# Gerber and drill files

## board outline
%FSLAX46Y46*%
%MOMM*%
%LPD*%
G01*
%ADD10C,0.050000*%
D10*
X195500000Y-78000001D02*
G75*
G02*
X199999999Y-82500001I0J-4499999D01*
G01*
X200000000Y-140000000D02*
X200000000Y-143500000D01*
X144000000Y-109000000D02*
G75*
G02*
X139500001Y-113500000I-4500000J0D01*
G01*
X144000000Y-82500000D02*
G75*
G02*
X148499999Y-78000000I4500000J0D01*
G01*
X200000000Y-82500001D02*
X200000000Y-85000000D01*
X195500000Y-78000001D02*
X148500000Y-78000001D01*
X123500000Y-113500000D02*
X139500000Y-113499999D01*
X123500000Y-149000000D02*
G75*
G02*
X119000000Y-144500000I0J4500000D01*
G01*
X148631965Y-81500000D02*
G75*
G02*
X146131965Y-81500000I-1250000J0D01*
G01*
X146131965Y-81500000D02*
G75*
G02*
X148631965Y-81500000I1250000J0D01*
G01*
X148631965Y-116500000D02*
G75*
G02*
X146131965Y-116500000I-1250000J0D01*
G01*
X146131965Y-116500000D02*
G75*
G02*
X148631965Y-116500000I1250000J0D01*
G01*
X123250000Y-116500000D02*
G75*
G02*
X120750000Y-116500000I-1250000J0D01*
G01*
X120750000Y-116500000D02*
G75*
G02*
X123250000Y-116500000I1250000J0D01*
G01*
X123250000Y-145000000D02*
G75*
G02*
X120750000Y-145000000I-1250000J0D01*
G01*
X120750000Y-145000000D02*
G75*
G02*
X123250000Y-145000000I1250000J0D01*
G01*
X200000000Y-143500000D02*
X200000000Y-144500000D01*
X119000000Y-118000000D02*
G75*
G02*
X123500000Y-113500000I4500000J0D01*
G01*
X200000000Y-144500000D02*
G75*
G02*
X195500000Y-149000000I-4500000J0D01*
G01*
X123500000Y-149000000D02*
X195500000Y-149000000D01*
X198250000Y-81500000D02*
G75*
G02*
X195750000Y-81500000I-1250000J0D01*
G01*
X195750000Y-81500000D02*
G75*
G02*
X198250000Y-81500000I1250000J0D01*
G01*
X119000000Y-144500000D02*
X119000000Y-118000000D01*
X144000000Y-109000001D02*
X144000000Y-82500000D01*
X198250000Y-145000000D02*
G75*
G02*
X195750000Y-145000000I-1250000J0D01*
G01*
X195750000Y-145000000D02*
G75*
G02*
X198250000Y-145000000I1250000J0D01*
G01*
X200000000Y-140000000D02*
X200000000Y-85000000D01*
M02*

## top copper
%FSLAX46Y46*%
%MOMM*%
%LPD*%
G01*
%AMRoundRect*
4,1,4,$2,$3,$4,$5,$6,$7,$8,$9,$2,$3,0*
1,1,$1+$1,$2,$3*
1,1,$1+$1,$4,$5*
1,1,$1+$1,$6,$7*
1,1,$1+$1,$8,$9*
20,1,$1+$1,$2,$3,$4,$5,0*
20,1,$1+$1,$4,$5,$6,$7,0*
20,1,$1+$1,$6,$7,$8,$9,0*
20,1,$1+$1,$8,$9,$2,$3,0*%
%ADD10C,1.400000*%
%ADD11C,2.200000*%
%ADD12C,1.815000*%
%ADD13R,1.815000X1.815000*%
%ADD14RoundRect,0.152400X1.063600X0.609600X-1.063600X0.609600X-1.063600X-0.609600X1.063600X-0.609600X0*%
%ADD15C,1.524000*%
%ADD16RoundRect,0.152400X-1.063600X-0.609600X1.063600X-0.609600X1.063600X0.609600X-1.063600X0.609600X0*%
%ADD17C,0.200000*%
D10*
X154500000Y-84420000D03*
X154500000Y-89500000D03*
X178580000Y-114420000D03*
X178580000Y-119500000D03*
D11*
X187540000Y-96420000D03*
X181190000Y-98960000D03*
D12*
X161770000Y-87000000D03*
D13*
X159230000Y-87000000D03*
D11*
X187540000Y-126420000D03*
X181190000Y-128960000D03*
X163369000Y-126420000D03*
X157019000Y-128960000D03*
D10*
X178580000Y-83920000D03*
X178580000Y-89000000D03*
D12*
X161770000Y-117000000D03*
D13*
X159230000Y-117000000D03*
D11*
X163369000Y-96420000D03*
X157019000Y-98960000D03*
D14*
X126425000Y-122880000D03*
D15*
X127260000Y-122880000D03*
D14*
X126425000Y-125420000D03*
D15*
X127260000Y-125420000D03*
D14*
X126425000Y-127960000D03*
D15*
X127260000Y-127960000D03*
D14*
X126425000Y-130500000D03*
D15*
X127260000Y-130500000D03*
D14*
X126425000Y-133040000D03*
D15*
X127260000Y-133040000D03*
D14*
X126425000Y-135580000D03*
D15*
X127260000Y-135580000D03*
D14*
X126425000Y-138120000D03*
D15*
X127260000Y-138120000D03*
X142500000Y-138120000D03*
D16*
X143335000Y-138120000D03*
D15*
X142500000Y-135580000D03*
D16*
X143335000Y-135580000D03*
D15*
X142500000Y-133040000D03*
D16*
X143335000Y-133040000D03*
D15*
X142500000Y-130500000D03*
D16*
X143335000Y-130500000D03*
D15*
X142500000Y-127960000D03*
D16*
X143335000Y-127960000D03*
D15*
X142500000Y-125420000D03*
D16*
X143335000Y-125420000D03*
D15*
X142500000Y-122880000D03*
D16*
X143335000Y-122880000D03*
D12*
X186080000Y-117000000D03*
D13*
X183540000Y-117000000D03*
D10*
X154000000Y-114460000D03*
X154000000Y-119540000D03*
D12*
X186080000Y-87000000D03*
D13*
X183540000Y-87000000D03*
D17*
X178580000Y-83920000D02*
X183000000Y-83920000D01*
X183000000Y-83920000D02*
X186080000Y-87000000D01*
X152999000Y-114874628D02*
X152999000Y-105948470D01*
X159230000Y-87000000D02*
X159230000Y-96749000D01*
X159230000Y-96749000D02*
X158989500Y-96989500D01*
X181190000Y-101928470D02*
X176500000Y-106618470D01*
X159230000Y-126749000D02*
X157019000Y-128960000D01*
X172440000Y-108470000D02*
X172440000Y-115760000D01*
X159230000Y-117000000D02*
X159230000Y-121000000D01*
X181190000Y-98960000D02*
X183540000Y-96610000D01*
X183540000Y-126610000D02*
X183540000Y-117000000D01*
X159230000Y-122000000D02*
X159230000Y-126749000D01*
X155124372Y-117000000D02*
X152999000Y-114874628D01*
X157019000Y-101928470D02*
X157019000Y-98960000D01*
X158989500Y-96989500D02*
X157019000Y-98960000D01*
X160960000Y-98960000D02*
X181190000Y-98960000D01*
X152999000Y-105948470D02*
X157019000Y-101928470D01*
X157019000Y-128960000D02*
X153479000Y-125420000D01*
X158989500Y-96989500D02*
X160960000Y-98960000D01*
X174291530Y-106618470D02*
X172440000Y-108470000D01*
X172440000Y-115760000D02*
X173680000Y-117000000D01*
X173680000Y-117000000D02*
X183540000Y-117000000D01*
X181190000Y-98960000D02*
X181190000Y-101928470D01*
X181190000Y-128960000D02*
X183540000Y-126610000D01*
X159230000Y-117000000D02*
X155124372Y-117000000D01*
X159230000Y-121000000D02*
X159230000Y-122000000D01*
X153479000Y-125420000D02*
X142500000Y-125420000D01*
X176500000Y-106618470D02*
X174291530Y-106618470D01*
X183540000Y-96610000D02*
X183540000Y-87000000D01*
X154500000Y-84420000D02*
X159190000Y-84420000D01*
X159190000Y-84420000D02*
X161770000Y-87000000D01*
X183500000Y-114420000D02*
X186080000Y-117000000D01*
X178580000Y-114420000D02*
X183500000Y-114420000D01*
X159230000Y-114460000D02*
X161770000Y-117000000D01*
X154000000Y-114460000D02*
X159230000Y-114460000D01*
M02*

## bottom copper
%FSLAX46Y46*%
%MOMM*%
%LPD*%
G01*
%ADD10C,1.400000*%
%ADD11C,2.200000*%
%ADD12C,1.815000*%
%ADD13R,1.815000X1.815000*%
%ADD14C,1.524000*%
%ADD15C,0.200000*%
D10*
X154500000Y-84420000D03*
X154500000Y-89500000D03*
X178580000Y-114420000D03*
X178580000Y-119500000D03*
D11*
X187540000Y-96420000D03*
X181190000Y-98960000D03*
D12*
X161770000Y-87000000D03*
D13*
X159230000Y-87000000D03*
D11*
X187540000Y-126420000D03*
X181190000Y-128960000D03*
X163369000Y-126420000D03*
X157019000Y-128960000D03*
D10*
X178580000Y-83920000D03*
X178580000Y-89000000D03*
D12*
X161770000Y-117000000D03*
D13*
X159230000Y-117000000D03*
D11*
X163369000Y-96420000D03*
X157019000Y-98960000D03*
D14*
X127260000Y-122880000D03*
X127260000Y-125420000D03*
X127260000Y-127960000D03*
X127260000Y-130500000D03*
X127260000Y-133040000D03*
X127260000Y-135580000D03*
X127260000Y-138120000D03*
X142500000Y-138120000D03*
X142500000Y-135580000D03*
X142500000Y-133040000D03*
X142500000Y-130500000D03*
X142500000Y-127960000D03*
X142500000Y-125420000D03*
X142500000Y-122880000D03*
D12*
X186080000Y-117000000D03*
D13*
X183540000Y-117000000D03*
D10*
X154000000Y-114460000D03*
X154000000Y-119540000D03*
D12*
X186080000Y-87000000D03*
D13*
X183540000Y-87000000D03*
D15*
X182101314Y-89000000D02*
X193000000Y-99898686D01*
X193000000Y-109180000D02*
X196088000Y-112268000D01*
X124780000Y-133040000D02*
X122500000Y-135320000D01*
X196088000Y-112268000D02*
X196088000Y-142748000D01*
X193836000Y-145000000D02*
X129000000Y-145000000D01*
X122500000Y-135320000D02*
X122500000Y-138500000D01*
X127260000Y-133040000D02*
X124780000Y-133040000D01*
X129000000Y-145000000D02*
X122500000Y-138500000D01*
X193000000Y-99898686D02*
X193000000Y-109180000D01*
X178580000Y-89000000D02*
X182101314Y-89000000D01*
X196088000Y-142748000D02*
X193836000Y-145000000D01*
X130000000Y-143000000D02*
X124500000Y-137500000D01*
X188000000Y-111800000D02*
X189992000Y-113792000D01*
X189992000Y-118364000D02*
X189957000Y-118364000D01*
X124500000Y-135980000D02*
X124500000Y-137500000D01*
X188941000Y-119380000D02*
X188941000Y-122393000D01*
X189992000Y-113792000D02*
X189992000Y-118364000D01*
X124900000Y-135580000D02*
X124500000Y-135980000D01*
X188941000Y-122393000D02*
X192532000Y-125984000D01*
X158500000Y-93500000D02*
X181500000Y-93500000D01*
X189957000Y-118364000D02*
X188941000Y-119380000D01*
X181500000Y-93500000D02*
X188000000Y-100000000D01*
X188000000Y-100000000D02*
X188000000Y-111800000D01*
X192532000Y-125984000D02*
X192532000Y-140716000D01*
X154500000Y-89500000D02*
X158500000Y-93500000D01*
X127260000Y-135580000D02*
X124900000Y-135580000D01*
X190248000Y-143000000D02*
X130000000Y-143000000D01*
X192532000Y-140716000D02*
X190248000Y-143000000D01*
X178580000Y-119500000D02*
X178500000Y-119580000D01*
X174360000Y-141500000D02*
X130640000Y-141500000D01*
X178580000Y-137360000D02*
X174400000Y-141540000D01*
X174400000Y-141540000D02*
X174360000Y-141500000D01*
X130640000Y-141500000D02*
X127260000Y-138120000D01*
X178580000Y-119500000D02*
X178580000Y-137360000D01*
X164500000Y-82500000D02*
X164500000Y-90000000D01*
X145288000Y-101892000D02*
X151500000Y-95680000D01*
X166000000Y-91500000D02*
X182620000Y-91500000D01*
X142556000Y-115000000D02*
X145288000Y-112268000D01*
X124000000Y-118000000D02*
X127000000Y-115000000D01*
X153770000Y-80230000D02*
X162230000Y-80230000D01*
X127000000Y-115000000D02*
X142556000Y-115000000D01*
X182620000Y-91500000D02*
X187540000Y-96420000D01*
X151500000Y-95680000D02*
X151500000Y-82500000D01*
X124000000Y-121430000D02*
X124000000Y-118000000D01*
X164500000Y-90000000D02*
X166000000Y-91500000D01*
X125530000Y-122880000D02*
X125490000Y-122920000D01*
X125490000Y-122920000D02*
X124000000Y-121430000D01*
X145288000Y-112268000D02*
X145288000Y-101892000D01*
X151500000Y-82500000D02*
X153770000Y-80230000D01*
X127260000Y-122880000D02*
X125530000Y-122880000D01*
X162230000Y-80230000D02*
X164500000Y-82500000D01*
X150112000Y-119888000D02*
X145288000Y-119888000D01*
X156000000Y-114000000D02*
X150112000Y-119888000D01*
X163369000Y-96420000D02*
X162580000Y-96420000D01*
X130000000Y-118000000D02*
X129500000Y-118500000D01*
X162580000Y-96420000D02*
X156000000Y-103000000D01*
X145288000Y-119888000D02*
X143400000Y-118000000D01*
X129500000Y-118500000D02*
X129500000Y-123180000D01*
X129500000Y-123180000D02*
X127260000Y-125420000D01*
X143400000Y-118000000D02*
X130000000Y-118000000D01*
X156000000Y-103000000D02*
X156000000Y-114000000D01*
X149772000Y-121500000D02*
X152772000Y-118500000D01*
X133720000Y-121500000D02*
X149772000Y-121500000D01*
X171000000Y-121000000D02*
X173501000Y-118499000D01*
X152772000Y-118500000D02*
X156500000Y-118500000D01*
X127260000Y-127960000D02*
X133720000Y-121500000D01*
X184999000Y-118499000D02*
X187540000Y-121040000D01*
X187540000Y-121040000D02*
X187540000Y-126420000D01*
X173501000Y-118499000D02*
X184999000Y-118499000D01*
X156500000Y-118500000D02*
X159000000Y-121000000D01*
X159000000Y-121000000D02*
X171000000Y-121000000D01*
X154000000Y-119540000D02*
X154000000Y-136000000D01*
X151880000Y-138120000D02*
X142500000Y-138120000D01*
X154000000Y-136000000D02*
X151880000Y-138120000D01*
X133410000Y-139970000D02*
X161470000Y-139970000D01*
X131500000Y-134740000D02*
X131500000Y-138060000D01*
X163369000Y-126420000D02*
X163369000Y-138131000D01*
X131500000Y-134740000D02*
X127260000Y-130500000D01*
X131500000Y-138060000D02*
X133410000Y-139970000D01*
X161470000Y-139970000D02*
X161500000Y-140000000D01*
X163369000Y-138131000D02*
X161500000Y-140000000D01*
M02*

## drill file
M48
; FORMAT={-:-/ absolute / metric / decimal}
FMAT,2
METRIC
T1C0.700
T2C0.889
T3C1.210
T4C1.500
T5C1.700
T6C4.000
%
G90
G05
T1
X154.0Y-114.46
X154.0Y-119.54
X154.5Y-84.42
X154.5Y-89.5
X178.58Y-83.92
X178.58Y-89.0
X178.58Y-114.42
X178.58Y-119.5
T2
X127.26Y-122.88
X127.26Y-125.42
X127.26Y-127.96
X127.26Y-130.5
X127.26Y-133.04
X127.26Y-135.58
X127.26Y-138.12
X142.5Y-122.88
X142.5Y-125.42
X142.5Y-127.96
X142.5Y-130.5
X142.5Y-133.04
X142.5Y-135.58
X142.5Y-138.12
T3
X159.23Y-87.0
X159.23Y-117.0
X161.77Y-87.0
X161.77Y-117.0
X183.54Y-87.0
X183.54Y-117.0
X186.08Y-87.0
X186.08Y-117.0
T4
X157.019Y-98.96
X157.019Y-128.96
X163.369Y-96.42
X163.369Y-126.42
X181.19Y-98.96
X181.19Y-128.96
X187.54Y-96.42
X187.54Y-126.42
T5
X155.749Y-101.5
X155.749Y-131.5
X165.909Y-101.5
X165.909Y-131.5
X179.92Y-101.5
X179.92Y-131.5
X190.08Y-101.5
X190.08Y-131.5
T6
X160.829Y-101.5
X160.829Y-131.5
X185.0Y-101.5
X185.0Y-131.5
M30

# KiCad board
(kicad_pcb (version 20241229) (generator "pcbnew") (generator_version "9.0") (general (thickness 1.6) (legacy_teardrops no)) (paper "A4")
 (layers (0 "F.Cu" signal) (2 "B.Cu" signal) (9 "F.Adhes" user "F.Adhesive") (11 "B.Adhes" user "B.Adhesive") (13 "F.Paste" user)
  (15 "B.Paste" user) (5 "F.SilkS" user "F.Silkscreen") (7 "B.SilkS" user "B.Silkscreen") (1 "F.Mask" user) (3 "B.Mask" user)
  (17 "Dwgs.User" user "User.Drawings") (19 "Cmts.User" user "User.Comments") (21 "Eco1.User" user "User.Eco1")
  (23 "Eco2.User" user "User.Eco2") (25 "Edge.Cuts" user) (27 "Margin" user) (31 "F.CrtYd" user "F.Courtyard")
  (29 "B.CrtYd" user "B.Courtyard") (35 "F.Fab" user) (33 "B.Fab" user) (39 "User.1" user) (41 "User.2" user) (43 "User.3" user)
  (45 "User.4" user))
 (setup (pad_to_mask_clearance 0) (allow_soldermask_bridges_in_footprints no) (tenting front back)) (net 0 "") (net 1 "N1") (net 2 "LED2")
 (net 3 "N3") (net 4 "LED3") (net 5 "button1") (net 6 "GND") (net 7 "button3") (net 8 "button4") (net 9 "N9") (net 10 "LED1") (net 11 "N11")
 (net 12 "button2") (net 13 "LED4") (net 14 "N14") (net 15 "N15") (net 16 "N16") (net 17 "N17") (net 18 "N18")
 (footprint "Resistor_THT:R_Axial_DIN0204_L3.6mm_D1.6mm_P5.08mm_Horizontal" (layer "F.Cu") (at 154.5 84.42 -90)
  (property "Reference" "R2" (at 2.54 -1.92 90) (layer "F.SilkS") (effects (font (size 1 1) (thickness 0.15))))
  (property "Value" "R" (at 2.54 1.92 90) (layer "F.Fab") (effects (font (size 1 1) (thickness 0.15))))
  (pad "1" thru_hole circle (at 0 0 270) (size 1.4 1.4) (drill 0.7) (layers "*.Cu" "*.Mask") (remove_unused_layers no) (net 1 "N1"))
  (pad "2" thru_hole circle (at 5.08 0 270) (size 1.4 1.4) (drill 0.7) (layers "*.Cu" "*.Mask") (remove_unused_layers no) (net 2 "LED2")))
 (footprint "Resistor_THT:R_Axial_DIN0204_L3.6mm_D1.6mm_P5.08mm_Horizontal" (layer "F.Cu") (at 178.58 114.42 -90)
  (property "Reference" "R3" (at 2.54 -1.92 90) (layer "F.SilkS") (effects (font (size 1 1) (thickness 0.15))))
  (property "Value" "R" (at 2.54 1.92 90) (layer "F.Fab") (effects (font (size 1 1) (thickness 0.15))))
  (pad "1" thru_hole circle (at 0 0 270) (size 1.4 1.4) (drill 0.7) (layers "*.Cu" "*.Mask") (remove_unused_layers no) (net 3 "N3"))
  (pad "2" thru_hole circle (at 5.08 0 270) (size 1.4 1.4) (drill 0.7) (layers "*.Cu" "*.Mask") (remove_unused_layers no) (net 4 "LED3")))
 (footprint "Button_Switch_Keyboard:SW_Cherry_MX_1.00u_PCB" (layer "F.Cu") (at 187.54 96.42)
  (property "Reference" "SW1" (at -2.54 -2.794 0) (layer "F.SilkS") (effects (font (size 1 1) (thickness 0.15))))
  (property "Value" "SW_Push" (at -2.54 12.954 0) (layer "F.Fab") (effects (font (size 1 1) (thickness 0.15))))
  (pad "" np_thru_hole circle (at -7.62 5.08) (size 1.7 1.7) (drill 1.7) (layers "*.Cu" "*.Mask"))
  (pad "" np_thru_hole circle (at -2.54 5.08) (size 4 4) (drill 4) (layers "*.Cu" "*.Mask"))
  (pad "" np_thru_hole circle (at 2.54 5.08) (size 1.7 1.7) (drill 1.7) (layers "*.Cu" "*.Mask"))
  (pad "1" thru_hole circle (at 0 0) (size 2.2 2.2) (drill 1.5) (layers "*.Cu" "*.Mask") (remove_unused_layers no) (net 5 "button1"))
  (pad "2" thru_hole circle (at -6.35 2.54) (size 2.2 2.2) (drill 1.5) (layers "*.Cu" "*.Mask") (remove_unused_layers no) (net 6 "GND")))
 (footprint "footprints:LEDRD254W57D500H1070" (layer "F.Cu") (at 160.5 87)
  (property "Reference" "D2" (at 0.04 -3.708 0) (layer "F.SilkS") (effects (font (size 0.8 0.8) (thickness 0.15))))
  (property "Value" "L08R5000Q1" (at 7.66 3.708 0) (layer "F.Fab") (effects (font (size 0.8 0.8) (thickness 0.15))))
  (pad "A" thru_hole circle (at 1.27 0) (size 1.815 1.815) (drill 1.21) (layers "*.Cu" "*.Mask") (remove_unused_layers no) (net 1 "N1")
   (solder_mask_margin 0.102))
  (pad "C" thru_hole rect (at -1.27 0) (size 1.815 1.815) (drill 1.21) (layers "*.Cu" "*.Mask") (remove_unused_layers no) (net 6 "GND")
   (solder_mask_margin 0.102)))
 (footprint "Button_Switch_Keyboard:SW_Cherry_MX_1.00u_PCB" (layer "F.Cu") (at 187.54 126.42)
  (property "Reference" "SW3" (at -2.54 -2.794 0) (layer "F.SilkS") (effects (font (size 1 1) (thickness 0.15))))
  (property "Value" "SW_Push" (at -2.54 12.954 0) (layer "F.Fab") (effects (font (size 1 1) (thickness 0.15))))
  (pad "" np_thru_hole circle (at -7.62 5.08) (size 1.7 1.7) (drill 1.7) (layers "*.Cu" "*.Mask"))
  (pad "" np_thru_hole circle (at -2.54 5.08) (size 4 4) (drill 4) (layers "*.Cu" "*.Mask"))
  (pad "" np_thru_hole circle (at 2.54 5.08) (size 1.7 1.7) (drill 1.7) (layers "*.Cu" "*.Mask"))
  (pad "1" thru_hole circle (at 0 0) (size 2.2 2.2) (drill 1.5) (layers "*.Cu" "*.Mask") (remove_unused_layers no) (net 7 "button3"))
  (pad "2" thru_hole circle (at -6.35 2.54) (size 2.2 2.2) (drill 1.5) (layers "*.Cu" "*.Mask") (remove_unused_layers no) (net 6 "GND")))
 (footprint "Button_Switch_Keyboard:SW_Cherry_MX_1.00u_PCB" (layer "F.Cu") (at 163.369 126.42)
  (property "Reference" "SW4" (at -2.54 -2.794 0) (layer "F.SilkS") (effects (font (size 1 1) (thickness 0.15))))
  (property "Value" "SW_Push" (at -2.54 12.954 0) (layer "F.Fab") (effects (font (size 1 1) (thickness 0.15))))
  (pad "" np_thru_hole circle (at -7.62 5.08) (size 1.7 1.7) (drill 1.7) (layers "*.Cu" "*.Mask"))
  (pad "" np_thru_hole circle (at -2.54 5.08) (size 4 4) (drill 4) (layers "*.Cu" "*.Mask"))
  (pad "" np_thru_hole circle (at 2.54 5.08) (size 1.7 1.7) (drill 1.7) (layers "*.Cu" "*.Mask"))
  (pad "1" thru_hole circle (at 0 0) (size 2.2 2.2) (drill 1.5) (layers "*.Cu" "*.Mask") (remove_unused_layers no) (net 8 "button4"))
  (pad "2" thru_hole circle (at -6.35 2.54) (size 2.2 2.2) (drill 1.5) (layers "*.Cu" "*.Mask") (remove_unused_layers no) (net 6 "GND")))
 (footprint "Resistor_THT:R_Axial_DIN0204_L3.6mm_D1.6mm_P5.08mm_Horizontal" (layer "F.Cu") (at 178.58 83.92 -90)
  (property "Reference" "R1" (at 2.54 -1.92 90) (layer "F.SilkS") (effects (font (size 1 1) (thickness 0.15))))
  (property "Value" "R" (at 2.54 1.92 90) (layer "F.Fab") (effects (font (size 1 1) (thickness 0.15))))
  (pad "1" thru_hole circle (at 0 0 270) (size 1.4 1.4) (drill 0.7) (layers "*.Cu" "*.Mask") (remove_unused_layers no) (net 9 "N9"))
  (pad "2" thru_hole circle (at 5.08 0 270) (size 1.4 1.4) (drill 0.7) (layers "*.Cu" "*.Mask") (remove_unused_layers no) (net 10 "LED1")))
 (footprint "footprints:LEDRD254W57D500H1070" (layer "F.Cu") (at 160.5 117)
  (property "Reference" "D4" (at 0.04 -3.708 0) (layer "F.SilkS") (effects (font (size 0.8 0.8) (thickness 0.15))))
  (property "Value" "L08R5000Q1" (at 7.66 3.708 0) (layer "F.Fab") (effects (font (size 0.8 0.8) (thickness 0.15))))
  (pad "A" thru_hole circle (at 1.27 0) (size 1.815 1.815) (drill 1.21) (layers "*.Cu" "*.Mask") (remove_unused_layers no) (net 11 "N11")
   (solder_mask_margin 0.102))
  (pad "C" thru_hole rect (at -1.27 0) (size 1.815 1.815) (drill 1.21) (layers "*.Cu" "*.Mask") (remove_unused_layers no) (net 6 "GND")
   (solder_mask_margin 0.102)))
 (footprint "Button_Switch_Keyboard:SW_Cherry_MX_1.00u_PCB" (layer "F.Cu") (at 163.369 96.42)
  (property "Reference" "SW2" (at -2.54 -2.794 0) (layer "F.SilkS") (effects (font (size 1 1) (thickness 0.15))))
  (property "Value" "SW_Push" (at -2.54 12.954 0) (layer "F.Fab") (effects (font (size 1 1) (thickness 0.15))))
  (pad "" np_thru_hole circle (at -7.62 5.08) (size 1.7 1.7) (drill 1.7) (layers "*.Cu" "*.Mask"))
  (pad "" np_thru_hole circle (at -2.54 5.08) (size 4 4) (drill 4) (layers "*.Cu" "*.Mask"))
  (pad "" np_thru_hole circle (at 2.54 5.08) (size 1.7 1.7) (drill 1.7) (layers "*.Cu" "*.Mask"))
  (pad "1" thru_hole circle (at 0 0) (size 2.2 2.2) (drill 1.5) (layers "*.Cu" "*.Mask") (remove_unused_layers no) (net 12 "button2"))
  (pad "2" thru_hole circle (at -6.35 2.54) (size 2.2 2.2) (drill 1.5) (layers "*.Cu" "*.Mask") (remove_unused_layers no) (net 6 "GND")))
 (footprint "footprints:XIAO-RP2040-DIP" (layer "F.Cu") (at 134.88 130.5)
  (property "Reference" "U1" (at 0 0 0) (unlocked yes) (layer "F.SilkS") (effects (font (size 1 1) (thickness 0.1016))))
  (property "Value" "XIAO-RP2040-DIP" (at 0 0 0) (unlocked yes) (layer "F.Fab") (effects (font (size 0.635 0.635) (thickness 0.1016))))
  (pad "1" smd roundrect (at -8.455 -7.62 180) (size 2.432 1.524) (layers "F.Cu" "F.Mask") (roundrect_rratio 0.1) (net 5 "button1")
   (thermal_bridge_angle 45))
  (pad "1" thru_hole circle (at -7.62 -7.62 180) (size 1.524 1.524) (drill 0.889) (layers "*.Cu" "*.Mask") (remove_unused_layers no)
   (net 5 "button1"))
  (pad "2" smd roundrect (at -8.455 -5.08 180) (size 2.432 1.524) (layers "F.Cu" "F.Mask") (roundrect_rratio 0.1) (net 12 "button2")
   (thermal_bridge_angle 45))
  (pad "2" thru_hole circle (at -7.62 -5.08 180) (size 1.524 1.524) (drill 0.889) (layers "*.Cu" "*.Mask") (remove_unused_layers no)
   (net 12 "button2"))
  (pad "3" smd roundrect (at -8.455 -2.54 180) (size 2.432 1.524) (layers "F.Cu" "F.Mask") (roundrect_rratio 0.1) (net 7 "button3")
   (thermal_bridge_angle 45))
  (pad "3" thru_hole circle (at -7.62 -2.54 180) (size 1.524 1.524) (drill 0.889) (layers "*.Cu" "*.Mask") (remove_unused_layers no)
   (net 7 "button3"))
  (pad "4" smd roundrect (at -8.455 0 180) (size 2.432 1.524) (layers "F.Cu" "F.Mask") (roundrect_rratio 0.1) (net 8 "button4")
   (thermal_bridge_angle 45))
  (pad "4" thru_hole circle (at -7.62 0 180) (size 1.524 1.524) (drill 0.889) (layers "*.Cu" "*.Mask") (remove_unused_layers no)
   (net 8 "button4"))
  (pad "5" smd roundrect (at -8.455 2.54 180) (size 2.432 1.524) (layers "F.Cu" "F.Mask") (roundrect_rratio 0.1) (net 10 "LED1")
   (thermal_bridge_angle 45))
  (pad "5" thru_hole circle (at -7.62 2.54 180) (size 1.524 1.524) (drill 0.889) (layers "*.Cu" "*.Mask") (remove_unused_layers no)
   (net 10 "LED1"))
  (pad "6" smd roundrect (at -8.455 5.08 180) (size 2.432 1.524) (layers "F.Cu" "F.Mask") (roundrect_rratio 0.1) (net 2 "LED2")
   (thermal_bridge_angle 45))
  (pad "6" thru_hole circle (at -7.62 5.08 180) (size 1.524 1.524) (drill 0.889) (layers "*.Cu" "*.Mask") (remove_unused_layers no)
   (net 2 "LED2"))
  (pad "7" smd roundrect (at -8.455 7.62 180) (size 2.432 1.524) (layers "F.Cu" "F.Mask") (roundrect_rratio 0.1) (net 4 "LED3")
   (thermal_bridge_angle 45))
  (pad "7" thru_hole circle (at -7.62 7.62 180) (size 1.524 1.524) (drill 0.889) (layers "*.Cu" "*.Mask") (remove_unused_layers no)
   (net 4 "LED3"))
  (pad "8" thru_hole circle (at 7.62 7.62) (size 1.524 1.524) (drill 0.889) (layers "*.Cu" "*.Mask") (remove_unused_layers no)
   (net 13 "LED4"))
  (pad "8" smd roundrect (at 8.455 7.62) (size 2.432 1.524) (layers "F.Cu" "F.Mask") (roundrect_rratio 0.1) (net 13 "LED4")
   (thermal_bridge_angle 45))
  (pad "9" thru_hole circle (at 7.62 5.08) (size 1.524 1.524) (drill 0.889) (layers "*.Cu" "*.Mask") (remove_unused_layers no)
   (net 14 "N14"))
  (pad "9" smd roundrect (at 8.455 5.08) (size 2.432 1.524) (layers "F.Cu" "F.Mask") (roundrect_rratio 0.1) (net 14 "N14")
   (thermal_bridge_angle 45))
  (pad "10" thru_hole circle (at 7.62 2.54) (size 1.524 1.524) (drill 0.889) (layers "*.Cu" "*.Mask") (remove_unused_layers no)
   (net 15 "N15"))
  (pad "10" smd roundrect (at 8.455 2.54) (size 2.432 1.524) (layers "F.Cu" "F.Mask") (roundrect_rratio 0.1) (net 15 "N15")
   (thermal_bridge_angle 45))
  (pad "11" thru_hole circle (at 7.62 0) (size 1.524 1.524) (drill 0.889) (layers "*.Cu" "*.Mask") (remove_unused_layers no) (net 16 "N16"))
  (pad "11" smd roundrect (at 8.455 0) (size 2.432 1.524) (layers "F.Cu" "F.Mask") (roundrect_rratio 0.1) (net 16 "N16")
   (thermal_bridge_angle 45))
  (pad "12" thru_hole circle (at 7.62 -2.54) (size 1.524 1.524) (drill 0.889) (layers "*.Cu" "*.Mask") (remove_unused_layers no)
   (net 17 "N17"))
  (pad "12" smd roundrect (at 8.455 -2.54) (size 2.432 1.524) (layers "F.Cu" "F.Mask") (roundrect_rratio 0.1) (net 17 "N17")
   (thermal_bridge_angle 45))
  (pad "13" thru_hole circle (at 7.62 -5.08) (size 1.524 1.524) (drill 0.889) (layers "*.Cu" "*.Mask") (remove_unused_layers no)
   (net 6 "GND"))
  (pad "13" smd roundrect (at 8.455 -5.08) (size 2.432 1.524) (layers "F.Cu" "F.Mask") (roundrect_rratio 0.1) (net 6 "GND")
   (thermal_bridge_angle 45))
  (pad "14" thru_hole circle (at 7.62 -7.62) (size 1.524 1.524) (drill 0.889) (layers "*.Cu" "*.Mask") (remove_unused_layers no)
   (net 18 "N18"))
  (pad "14" smd roundrect (at 8.455 -7.62) (size 2.432 1.524) (layers "F.Cu" "F.Mask") (roundrect_rratio 0.1) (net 18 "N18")
   (thermal_bridge_angle 45)))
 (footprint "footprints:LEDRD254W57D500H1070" (layer "F.Cu") (at 184.81 117)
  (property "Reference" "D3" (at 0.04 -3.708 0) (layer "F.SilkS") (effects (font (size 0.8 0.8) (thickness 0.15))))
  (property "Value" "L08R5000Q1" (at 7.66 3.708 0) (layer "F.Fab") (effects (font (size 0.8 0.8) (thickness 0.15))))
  (pad "A" thru_hole circle (at 1.27 0) (size 1.815 1.815) (drill 1.21) (layers "*.Cu" "*.Mask") (remove_unused_layers no) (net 3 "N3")
   (solder_mask_margin 0.102))
  (pad "C" thru_hole rect (at -1.27 0) (size 1.815 1.815) (drill 1.21) (layers "*.Cu" "*.Mask") (remove_unused_layers no) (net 6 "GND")
   (solder_mask_margin 0.102)))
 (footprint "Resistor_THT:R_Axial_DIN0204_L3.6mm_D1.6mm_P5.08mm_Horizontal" (layer "F.Cu") (at 154 114.46 -90)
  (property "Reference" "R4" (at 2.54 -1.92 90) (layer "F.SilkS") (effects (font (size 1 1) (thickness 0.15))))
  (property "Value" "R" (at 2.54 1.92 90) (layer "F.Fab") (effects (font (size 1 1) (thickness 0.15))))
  (pad "1" thru_hole circle (at 0 0 270) (size 1.4 1.4) (drill 0.7) (layers "*.Cu" "*.Mask") (remove_unused_layers no) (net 11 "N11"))
  (pad "2" thru_hole circle (at 5.08 0 270) (size 1.4 1.4) (drill 0.7) (layers "*.Cu" "*.Mask") (remove_unused_layers no) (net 13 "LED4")))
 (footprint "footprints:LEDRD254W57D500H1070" (layer "F.Cu") (at 184.81 87)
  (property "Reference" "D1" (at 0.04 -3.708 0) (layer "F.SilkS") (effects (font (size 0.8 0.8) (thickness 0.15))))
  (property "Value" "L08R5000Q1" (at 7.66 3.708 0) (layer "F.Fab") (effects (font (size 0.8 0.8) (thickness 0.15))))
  (pad "A" thru_hole circle (at 1.27 0) (size 1.815 1.815) (drill 1.21) (layers "*.Cu" "*.Mask") (remove_unused_layers no) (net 9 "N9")
   (solder_mask_margin 0.102))
  (pad "C" thru_hole rect (at -1.27 0) (size 1.815 1.815) (drill 1.21) (layers "*.Cu" "*.Mask") (remove_unused_layers no) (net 6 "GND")
   (solder_mask_margin 0.102)))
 (gr_arc (start 195.5 78.000001) (mid 198.681981 79.31802) (end 200 82.500001) (stroke (width 0.05) (type default)) (layer "Edge.Cuts"))
 (gr_line (start 200 140) (end 200 143.5) (stroke (width 0.05) (type default)) (layer "Edge.Cuts"))
 (gr_arc (start 144 109) (mid 142.681982 112.181986) (end 139.500001 113.499999) (stroke (width 0.05) (type default)) (layer "Edge.Cuts"))
 (gr_arc (start 144 82.5) (mid 145.31802 79.318026) (end 148.499999 78.000001) (stroke (width 0.05) (type default)) (layer "Edge.Cuts"))
 (gr_line (start 200 82.500001) (end 200 85) (stroke (width 0.05) (type default)) (layer "Edge.Cuts"))
 (gr_line (start 195.5 78.000001) (end 148.5 78.000001) (stroke (width 0.05) (type default)) (layer "Edge.Cuts"))
 (gr_line (start 123.5 113.5) (end 139.5 113.499999) (stroke (width 0.05) (type default)) (layer "Edge.Cuts"))
 (gr_arc (start 123.5 149) (mid 120.318019 147.681981) (end 119 144.5) (stroke (width 0.05) (type default)) (layer "Edge.Cuts"))
 (gr_circle (center 147.381965 81.5) (end 148.631965 81.5) (stroke (width 0.05) (type solid)) (fill no) (layer "Edge.Cuts"))
 (gr_circle (center 147.381965 116.5) (end 148.631965 116.5) (stroke (width 0.05) (type solid)) (fill no) (layer "Edge.Cuts"))
 (gr_circle (center 122 116.5) (end 123.25 116.5) (stroke (width 0.05) (type solid)) (fill no) (layer "Edge.Cuts"))
 (gr_circle (center 122 145) (end 123.25 145) (stroke (width 0.05) (type solid)) (fill no) (layer "Edge.Cuts"))
 (gr_line (start 200 143.5) (end 200 144.5) (stroke (width 0.05) (type default)) (layer "Edge.Cuts"))
 (gr_arc (start 119 118) (mid 120.31802 114.81802) (end 123.5 113.5) (stroke (width 0.05) (type default)) (layer "Edge.Cuts"))
 (gr_arc (start 200 144.5) (mid 198.681981 147.681981) (end 195.5 149) (stroke (width 0.05) (type default)) (layer "Edge.Cuts"))
 (gr_line (start 123.5 149) (end 195.5 149) (stroke (width 0.05) (type default)) (layer "Edge.Cuts"))
 (gr_circle (center 197 81.5) (end 198.25 81.5) (stroke (width 0.05) (type solid)) (fill no) (layer "Edge.Cuts"))
 (gr_line (start 119 144.5) (end 119 118) (stroke (width 0.05) (type default)) (layer "Edge.Cuts"))
 (gr_line (start 144 109.000001) (end 144 82.5) (stroke (width 0.05) (type default)) (layer "Edge.Cuts"))
 (gr_circle (center 197 145) (end 198.25 145) (stroke (width 0.05) (type solid)) (fill no) (layer "Edge.Cuts"))
 (gr_line (start 200 140) (end 200 85) (stroke (width 0.05) (type solid)) (layer "Edge.Cuts"))
 (segment (start 178.58 83.92) (end 183 83.92) (width 0.2) (layer "F.Cu") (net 9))
 (segment (start 183 83.92) (end 186.08 87) (width 0.2) (layer "F.Cu") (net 9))
 (segment (start 152.999 114.874628) (end 152.999 105.94847) (width 0.2) (layer "F.Cu") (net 6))
 (segment (start 159.23 87) (end 159.23 96.749) (width 0.2) (layer "F.Cu") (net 6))
 (segment (start 159.23 96.749) (end 158.9895 96.9895) (width 0.2) (layer "F.Cu") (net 6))
 (segment (start 181.19 101.92847) (end 176.5 106.61847) (width 0.2) (layer "F.Cu") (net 6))
 (segment (start 159.23 126.749) (end 157.019 128.96) (width 0.2) (layer "F.Cu") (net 6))
 (segment (start 172.44 108.47) (end 172.44 115.76) (width 0.2) (layer "F.Cu") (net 6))
 (segment (start 159.23 117) (end 159.23 121) (width 0.2) (layer "F.Cu") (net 6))
 (segment (start 181.19 98.96) (end 183.54 96.61) (width 0.2) (layer "F.Cu") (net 6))
 (segment (start 183.54 126.61) (end 183.54 117) (width 0.2) (layer "F.Cu") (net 6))
 (segment (start 159.23 122) (end 159.23 126.749) (width 0.2) (layer "F.Cu") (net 6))
 (segment (start 155.124372 117) (end 152.999 114.874628) (width 0.2) (layer "F.Cu") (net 6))
 (segment (start 157.019 101.92847) (end 157.019 98.96) (width 0.2) (layer "F.Cu") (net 6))
 (segment (start 158.9895 96.9895) (end 157.019 98.96) (width 0.2) (layer "F.Cu") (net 6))
 (segment (start 160.96 98.96) (end 181.19 98.96) (width 0.2) (layer "F.Cu") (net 6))
 (segment (start 152.999 105.94847) (end 157.019 101.92847) (width 0.2) (layer "F.Cu") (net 6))
 (segment (start 157.019 128.96) (end 153.479 125.42) (width 0.2) (layer "F.Cu") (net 6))
 (segment (start 158.9895 96.9895) (end 160.96 98.96) (width 0.2) (layer "F.Cu") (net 6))
 (segment (start 174.29153 106.61847) (end 172.44 108.47) (width 0.2) (layer "F.Cu") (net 6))
 (segment (start 172.44 115.76) (end 173.68 117) (width 0.2) (layer "F.Cu") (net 6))
 (segment (start 173.68 117) (end 183.54 117) (width 0.2) (layer "F.Cu") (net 6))
 (segment (start 181.19 98.96) (end 181.19 101.92847) (width 0.2) (layer "F.Cu") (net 6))
 (segment (start 181.19 128.96) (end 183.54 126.61) (width 0.2) (layer "F.Cu") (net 6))
 (segment (start 159.23 117) (end 155.124372 117) (width 0.2) (layer "F.Cu") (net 6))
 (segment (start 159.23 121) (end 159.23 122) (width 0.2) (layer "F.Cu") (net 6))
 (segment (start 153.479 125.42) (end 142.5 125.42) (width 0.2) (layer "F.Cu") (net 6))
 (segment (start 176.5 106.61847) (end 174.29153 106.61847) (width 0.2) (layer "F.Cu") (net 6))
 (segment (start 183.54 96.61) (end 183.54 87) (width 0.2) (layer "F.Cu") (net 6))
 (segment (start 154.5 84.42) (end 159.19 84.42) (width 0.2) (layer "F.Cu") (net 1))
 (segment (start 159.19 84.42) (end 161.77 87) (width 0.2) (layer "F.Cu") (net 1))
 (segment (start 183.5 114.42) (end 186.08 117) (width 0.2) (layer "F.Cu") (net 3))
 (segment (start 178.58 114.42) (end 183.5 114.42) (width 0.2) (layer "F.Cu") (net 3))
 (segment (start 182.101314 89) (end 193 99.898686) (width 0.2) (layer "B.Cu") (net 10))
 (segment (start 193 109.18) (end 196.088 112.268) (width 0.2) (layer "B.Cu") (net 10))
 (segment (start 124.78 133.04) (end 122.5 135.32) (width 0.2) (layer "B.Cu") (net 10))
 (segment (start 196.088 112.268) (end 196.088 142.748) (width 0.2) (layer "B.Cu") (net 10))
 (segment (start 193.836 145) (end 129 145) (width 0.2) (layer "B.Cu") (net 10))
 (segment (start 122.5 135.32) (end 122.5 138.5) (width 0.2) (layer "B.Cu") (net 10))
 (segment (start 127.26 133.04) (end 124.78 133.04) (width 0.2) (layer "B.Cu") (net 10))
 (segment (start 129 145) (end 122.5 138.5) (width 0.2) (layer "B.Cu") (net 10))
 (segment (start 193 99.898686) (end 193 109.18) (width 0.2) (layer "B.Cu") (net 10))
 (segment (start 178.58 89) (end 182.101314 89) (width 0.2) (layer "B.Cu") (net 10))
 (segment (start 196.088 142.748) (end 193.836 145) (width 0.2) (layer "B.Cu") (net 10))
 (segment (start 130 143) (end 124.5 137.5) (width 0.2) (layer "B.Cu") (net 2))
 (segment (start 188 111.8) (end 189.992 113.792) (width 0.2) (layer "B.Cu") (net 2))
 (segment (start 189.992 118.364) (end 189.957 118.364) (width 0.2) (layer "B.Cu") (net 2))
 (segment (start 124.5 135.98) (end 124.5 137.5) (width 0.2) (layer "B.Cu") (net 2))
 (segment (start 188.941 119.38) (end 188.941 122.393) (width 0.2) (layer "B.Cu") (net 2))
 (segment (start 189.992 113.792) (end 189.992 118.364) (width 0.2) (layer "B.Cu") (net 2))
 (segment (start 124.9 135.58) (end 124.5 135.98) (width 0.2) (layer "B.Cu") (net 2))
 (segment (start 188.941 122.393) (end 192.532 125.984) (width 0.2) (layer "B.Cu") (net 2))
 (segment (start 158.5 93.5) (end 181.5 93.5) (width 0.2) (layer "B.Cu") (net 2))
 (segment (start 189.957 118.364) (end 188.941 119.38) (width 0.2) (layer "B.Cu") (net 2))
 (segment (start 181.5 93.5) (end 188 100) (width 0.2) (layer "B.Cu") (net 2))
 (segment (start 188 100) (end 188 111.8) (width 0.2) (layer "B.Cu") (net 2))
 (segment (start 192.532 125.984) (end 192.532 140.716) (width 0.2) (layer "B.Cu") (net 2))
 (segment (start 154.5 89.5) (end 158.5 93.5) (width 0.2) (layer "B.Cu") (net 2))
 (segment (start 127.26 135.58) (end 124.9 135.58) (width 0.2) (layer "B.Cu") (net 2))
 (segment (start 190.248 143) (end 130 143) (width 0.2) (layer "B.Cu") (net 2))
 (segment (start 192.532 140.716) (end 190.248 143) (width 0.2) (layer "B.Cu") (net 2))
 (segment (start 178.58 119.5) (end 178.5 119.58) (width 0.2) (layer "B.Cu") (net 4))
 (segment (start 174.36 141.5) (end 130.64 141.5) (width 0.2) (layer "B.Cu") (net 4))
 (segment (start 178.58 137.36) (end 174.4 141.54) (width 0.2) (layer "B.Cu") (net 4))
 (segment (start 174.4 141.54) (end 174.36 141.5) (width 0.2) (layer "B.Cu") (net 4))
 (segment (start 130.64 141.5) (end 127.26 138.12) (width 0.2) (layer "B.Cu") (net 4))
 (segment (start 178.58 119.5) (end 178.58 137.36) (width 0.2) (layer "B.Cu") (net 4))
 (segment (start 164.5 82.5) (end 164.5 90) (width 0.2) (layer "B.Cu") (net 5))
 (segment (start 145.288 101.892) (end 151.5 95.68) (width 0.2) (layer "B.Cu") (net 5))
 (segment (start 166 91.5) (end 182.62 91.5) (width 0.2) (layer "B.Cu") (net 5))
 (segment (start 142.556 115) (end 145.288 112.268) (width 0.2) (layer "B.Cu") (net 5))
 (segment (start 124 118) (end 127 115) (width 0.2) (layer "B.Cu") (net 5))
 (segment (start 153.77 80.23) (end 162.23 80.23) (width 0.2) (layer "B.Cu") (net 5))
 (segment (start 127 115) (end 142.556 115) (width 0.2) (layer "B.Cu") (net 5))
 (segment (start 182.62 91.5) (end 187.54 96.42) (width 0.2) (layer "B.Cu") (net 5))
 (segment (start 151.5 95.68) (end 151.5 82.5) (width 0.2) (layer "B.Cu") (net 5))
 (segment (start 124 121.43) (end 124 118) (width 0.2) (layer "B.Cu") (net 5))
 (segment (start 164.5 90) (end 166 91.5) (width 0.2) (layer "B.Cu") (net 5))
 (segment (start 125.53 122.88) (end 125.49 122.92) (width 0.2) (layer "B.Cu") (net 5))
 (segment (start 125.49 122.92) (end 124 121.43) (width 0.2) (layer "B.Cu") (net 5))
 (segment (start 145.288 112.268) (end 145.288 101.892) (width 0.2) (layer "B.Cu") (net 5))
 (segment (start 151.5 82.5) (end 153.77 80.23) (width 0.2) (layer "B.Cu") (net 5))
 (segment (start 127.26 122.88) (end 125.53 122.88) (width 0.2) (layer "B.Cu") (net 5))
 (segment (start 162.23 80.23) (end 164.5 82.5) (width 0.2) (layer "B.Cu") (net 5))
 (segment (start 150.112 119.888) (end 145.288 119.888) (width 0.2) (layer "B.Cu") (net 12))
 (segment (start 156 114) (end 150.112 119.888) (width 0.2) (layer "B.Cu") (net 12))
 (segment (start 163.369 96.42) (end 162.58 96.42) (width 0.2) (layer "B.Cu") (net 12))
 (segment (start 130 118) (end 129.5 118.5) (width 0.2) (layer "B.Cu") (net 12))
 (segment (start 162.58 96.42) (end 156 103) (width 0.2) (layer "B.Cu") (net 12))
 (segment (start 145.288 119.888) (end 143.4 118) (width 0.2) (layer "B.Cu") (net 12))
 (segment (start 129.5 118.5) (end 129.5 123.18) (width 0.2) (layer "B.Cu") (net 12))
 (segment (start 129.5 123.18) (end 127.26 125.42) (width 0.2) (layer "B.Cu") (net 12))
 (segment (start 143.4 118) (end 130 118) (width 0.2) (layer "B.Cu") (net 12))
 (segment (start 156 103) (end 156 114) (width 0.2) (layer "B.Cu") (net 12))
 (segment (start 149.772 121.5) (end 152.772 118.5) (width 0.2) (layer "B.Cu") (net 7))
 (segment (start 133.72 121.5) (end 149.772 121.5) (width 0.2) (layer "B.Cu") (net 7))
 (segment (start 171 121) (end 173.501 118.499) (width 0.2) (layer "B.Cu") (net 7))
 (segment (start 152.772 118.5) (end 156.5 118.5) (width 0.2) (layer "B.Cu") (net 7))
 (segment (start 127.26 127.96) (end 133.72 121.5) (width 0.2) (layer "B.Cu") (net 7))
 (segment (start 184.999 118.499) (end 187.54 121.04) (width 0.2) (layer "B.Cu") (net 7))
 (segment (start 187.54 121.04) (end 187.54 126.42) (width 0.2) (layer "B.Cu") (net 7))
 (segment (start 173.501 118.499) (end 184.999 118.499) (width 0.2) (layer "B.Cu") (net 7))
 (segment (start 156.5 118.5) (end 159 121) (width 0.2) (layer "B.Cu") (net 7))
 (segment (start 159 121) (end 171 121) (width 0.2) (layer "B.Cu") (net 7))
 (segment (start 159.23 114.46) (end 161.77 117) (width 0.2) (layer "F.Cu") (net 11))
 (segment (start 154 114.46) (end 159.23 114.46) (width 0.2) (layer "F.Cu") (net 11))
 (segment (start 154 119.54) (end 154 136) (width 0.2) (layer "B.Cu") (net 13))
 (segment (start 151.88 138.12) (end 142.5 138.12) (width 0.2) (layer "B.Cu") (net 13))
 (segment (start 154 136) (end 151.88 138.12) (width 0.2) (layer "B.Cu") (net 13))
 (segment (start 133.41 139.97) (end 161.47 139.97) (width 0.2) (layer "B.Cu") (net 8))
 (segment (start 131.5 134.74) (end 131.5 138.06) (width 0.2) (layer "B.Cu") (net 8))
 (segment (start 163.369 126.42) (end 163.369 138.131) (width 0.2) (layer "B.Cu") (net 8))
 (segment (start 131.5 134.74) (end 127.26 130.5) (width 0.2) (layer "B.Cu") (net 8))
 (segment (start 131.5 138.06) (end 133.41 139.97) (width 0.2) (layer "B.Cu") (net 8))
 (segment (start 161.47 139.97) (end 161.5 140) (width 0.2) (layer "B.Cu") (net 8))
 (segment (start 163.369 138.131) (end 161.5 140) (width 0.2) (layer "B.Cu") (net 8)))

